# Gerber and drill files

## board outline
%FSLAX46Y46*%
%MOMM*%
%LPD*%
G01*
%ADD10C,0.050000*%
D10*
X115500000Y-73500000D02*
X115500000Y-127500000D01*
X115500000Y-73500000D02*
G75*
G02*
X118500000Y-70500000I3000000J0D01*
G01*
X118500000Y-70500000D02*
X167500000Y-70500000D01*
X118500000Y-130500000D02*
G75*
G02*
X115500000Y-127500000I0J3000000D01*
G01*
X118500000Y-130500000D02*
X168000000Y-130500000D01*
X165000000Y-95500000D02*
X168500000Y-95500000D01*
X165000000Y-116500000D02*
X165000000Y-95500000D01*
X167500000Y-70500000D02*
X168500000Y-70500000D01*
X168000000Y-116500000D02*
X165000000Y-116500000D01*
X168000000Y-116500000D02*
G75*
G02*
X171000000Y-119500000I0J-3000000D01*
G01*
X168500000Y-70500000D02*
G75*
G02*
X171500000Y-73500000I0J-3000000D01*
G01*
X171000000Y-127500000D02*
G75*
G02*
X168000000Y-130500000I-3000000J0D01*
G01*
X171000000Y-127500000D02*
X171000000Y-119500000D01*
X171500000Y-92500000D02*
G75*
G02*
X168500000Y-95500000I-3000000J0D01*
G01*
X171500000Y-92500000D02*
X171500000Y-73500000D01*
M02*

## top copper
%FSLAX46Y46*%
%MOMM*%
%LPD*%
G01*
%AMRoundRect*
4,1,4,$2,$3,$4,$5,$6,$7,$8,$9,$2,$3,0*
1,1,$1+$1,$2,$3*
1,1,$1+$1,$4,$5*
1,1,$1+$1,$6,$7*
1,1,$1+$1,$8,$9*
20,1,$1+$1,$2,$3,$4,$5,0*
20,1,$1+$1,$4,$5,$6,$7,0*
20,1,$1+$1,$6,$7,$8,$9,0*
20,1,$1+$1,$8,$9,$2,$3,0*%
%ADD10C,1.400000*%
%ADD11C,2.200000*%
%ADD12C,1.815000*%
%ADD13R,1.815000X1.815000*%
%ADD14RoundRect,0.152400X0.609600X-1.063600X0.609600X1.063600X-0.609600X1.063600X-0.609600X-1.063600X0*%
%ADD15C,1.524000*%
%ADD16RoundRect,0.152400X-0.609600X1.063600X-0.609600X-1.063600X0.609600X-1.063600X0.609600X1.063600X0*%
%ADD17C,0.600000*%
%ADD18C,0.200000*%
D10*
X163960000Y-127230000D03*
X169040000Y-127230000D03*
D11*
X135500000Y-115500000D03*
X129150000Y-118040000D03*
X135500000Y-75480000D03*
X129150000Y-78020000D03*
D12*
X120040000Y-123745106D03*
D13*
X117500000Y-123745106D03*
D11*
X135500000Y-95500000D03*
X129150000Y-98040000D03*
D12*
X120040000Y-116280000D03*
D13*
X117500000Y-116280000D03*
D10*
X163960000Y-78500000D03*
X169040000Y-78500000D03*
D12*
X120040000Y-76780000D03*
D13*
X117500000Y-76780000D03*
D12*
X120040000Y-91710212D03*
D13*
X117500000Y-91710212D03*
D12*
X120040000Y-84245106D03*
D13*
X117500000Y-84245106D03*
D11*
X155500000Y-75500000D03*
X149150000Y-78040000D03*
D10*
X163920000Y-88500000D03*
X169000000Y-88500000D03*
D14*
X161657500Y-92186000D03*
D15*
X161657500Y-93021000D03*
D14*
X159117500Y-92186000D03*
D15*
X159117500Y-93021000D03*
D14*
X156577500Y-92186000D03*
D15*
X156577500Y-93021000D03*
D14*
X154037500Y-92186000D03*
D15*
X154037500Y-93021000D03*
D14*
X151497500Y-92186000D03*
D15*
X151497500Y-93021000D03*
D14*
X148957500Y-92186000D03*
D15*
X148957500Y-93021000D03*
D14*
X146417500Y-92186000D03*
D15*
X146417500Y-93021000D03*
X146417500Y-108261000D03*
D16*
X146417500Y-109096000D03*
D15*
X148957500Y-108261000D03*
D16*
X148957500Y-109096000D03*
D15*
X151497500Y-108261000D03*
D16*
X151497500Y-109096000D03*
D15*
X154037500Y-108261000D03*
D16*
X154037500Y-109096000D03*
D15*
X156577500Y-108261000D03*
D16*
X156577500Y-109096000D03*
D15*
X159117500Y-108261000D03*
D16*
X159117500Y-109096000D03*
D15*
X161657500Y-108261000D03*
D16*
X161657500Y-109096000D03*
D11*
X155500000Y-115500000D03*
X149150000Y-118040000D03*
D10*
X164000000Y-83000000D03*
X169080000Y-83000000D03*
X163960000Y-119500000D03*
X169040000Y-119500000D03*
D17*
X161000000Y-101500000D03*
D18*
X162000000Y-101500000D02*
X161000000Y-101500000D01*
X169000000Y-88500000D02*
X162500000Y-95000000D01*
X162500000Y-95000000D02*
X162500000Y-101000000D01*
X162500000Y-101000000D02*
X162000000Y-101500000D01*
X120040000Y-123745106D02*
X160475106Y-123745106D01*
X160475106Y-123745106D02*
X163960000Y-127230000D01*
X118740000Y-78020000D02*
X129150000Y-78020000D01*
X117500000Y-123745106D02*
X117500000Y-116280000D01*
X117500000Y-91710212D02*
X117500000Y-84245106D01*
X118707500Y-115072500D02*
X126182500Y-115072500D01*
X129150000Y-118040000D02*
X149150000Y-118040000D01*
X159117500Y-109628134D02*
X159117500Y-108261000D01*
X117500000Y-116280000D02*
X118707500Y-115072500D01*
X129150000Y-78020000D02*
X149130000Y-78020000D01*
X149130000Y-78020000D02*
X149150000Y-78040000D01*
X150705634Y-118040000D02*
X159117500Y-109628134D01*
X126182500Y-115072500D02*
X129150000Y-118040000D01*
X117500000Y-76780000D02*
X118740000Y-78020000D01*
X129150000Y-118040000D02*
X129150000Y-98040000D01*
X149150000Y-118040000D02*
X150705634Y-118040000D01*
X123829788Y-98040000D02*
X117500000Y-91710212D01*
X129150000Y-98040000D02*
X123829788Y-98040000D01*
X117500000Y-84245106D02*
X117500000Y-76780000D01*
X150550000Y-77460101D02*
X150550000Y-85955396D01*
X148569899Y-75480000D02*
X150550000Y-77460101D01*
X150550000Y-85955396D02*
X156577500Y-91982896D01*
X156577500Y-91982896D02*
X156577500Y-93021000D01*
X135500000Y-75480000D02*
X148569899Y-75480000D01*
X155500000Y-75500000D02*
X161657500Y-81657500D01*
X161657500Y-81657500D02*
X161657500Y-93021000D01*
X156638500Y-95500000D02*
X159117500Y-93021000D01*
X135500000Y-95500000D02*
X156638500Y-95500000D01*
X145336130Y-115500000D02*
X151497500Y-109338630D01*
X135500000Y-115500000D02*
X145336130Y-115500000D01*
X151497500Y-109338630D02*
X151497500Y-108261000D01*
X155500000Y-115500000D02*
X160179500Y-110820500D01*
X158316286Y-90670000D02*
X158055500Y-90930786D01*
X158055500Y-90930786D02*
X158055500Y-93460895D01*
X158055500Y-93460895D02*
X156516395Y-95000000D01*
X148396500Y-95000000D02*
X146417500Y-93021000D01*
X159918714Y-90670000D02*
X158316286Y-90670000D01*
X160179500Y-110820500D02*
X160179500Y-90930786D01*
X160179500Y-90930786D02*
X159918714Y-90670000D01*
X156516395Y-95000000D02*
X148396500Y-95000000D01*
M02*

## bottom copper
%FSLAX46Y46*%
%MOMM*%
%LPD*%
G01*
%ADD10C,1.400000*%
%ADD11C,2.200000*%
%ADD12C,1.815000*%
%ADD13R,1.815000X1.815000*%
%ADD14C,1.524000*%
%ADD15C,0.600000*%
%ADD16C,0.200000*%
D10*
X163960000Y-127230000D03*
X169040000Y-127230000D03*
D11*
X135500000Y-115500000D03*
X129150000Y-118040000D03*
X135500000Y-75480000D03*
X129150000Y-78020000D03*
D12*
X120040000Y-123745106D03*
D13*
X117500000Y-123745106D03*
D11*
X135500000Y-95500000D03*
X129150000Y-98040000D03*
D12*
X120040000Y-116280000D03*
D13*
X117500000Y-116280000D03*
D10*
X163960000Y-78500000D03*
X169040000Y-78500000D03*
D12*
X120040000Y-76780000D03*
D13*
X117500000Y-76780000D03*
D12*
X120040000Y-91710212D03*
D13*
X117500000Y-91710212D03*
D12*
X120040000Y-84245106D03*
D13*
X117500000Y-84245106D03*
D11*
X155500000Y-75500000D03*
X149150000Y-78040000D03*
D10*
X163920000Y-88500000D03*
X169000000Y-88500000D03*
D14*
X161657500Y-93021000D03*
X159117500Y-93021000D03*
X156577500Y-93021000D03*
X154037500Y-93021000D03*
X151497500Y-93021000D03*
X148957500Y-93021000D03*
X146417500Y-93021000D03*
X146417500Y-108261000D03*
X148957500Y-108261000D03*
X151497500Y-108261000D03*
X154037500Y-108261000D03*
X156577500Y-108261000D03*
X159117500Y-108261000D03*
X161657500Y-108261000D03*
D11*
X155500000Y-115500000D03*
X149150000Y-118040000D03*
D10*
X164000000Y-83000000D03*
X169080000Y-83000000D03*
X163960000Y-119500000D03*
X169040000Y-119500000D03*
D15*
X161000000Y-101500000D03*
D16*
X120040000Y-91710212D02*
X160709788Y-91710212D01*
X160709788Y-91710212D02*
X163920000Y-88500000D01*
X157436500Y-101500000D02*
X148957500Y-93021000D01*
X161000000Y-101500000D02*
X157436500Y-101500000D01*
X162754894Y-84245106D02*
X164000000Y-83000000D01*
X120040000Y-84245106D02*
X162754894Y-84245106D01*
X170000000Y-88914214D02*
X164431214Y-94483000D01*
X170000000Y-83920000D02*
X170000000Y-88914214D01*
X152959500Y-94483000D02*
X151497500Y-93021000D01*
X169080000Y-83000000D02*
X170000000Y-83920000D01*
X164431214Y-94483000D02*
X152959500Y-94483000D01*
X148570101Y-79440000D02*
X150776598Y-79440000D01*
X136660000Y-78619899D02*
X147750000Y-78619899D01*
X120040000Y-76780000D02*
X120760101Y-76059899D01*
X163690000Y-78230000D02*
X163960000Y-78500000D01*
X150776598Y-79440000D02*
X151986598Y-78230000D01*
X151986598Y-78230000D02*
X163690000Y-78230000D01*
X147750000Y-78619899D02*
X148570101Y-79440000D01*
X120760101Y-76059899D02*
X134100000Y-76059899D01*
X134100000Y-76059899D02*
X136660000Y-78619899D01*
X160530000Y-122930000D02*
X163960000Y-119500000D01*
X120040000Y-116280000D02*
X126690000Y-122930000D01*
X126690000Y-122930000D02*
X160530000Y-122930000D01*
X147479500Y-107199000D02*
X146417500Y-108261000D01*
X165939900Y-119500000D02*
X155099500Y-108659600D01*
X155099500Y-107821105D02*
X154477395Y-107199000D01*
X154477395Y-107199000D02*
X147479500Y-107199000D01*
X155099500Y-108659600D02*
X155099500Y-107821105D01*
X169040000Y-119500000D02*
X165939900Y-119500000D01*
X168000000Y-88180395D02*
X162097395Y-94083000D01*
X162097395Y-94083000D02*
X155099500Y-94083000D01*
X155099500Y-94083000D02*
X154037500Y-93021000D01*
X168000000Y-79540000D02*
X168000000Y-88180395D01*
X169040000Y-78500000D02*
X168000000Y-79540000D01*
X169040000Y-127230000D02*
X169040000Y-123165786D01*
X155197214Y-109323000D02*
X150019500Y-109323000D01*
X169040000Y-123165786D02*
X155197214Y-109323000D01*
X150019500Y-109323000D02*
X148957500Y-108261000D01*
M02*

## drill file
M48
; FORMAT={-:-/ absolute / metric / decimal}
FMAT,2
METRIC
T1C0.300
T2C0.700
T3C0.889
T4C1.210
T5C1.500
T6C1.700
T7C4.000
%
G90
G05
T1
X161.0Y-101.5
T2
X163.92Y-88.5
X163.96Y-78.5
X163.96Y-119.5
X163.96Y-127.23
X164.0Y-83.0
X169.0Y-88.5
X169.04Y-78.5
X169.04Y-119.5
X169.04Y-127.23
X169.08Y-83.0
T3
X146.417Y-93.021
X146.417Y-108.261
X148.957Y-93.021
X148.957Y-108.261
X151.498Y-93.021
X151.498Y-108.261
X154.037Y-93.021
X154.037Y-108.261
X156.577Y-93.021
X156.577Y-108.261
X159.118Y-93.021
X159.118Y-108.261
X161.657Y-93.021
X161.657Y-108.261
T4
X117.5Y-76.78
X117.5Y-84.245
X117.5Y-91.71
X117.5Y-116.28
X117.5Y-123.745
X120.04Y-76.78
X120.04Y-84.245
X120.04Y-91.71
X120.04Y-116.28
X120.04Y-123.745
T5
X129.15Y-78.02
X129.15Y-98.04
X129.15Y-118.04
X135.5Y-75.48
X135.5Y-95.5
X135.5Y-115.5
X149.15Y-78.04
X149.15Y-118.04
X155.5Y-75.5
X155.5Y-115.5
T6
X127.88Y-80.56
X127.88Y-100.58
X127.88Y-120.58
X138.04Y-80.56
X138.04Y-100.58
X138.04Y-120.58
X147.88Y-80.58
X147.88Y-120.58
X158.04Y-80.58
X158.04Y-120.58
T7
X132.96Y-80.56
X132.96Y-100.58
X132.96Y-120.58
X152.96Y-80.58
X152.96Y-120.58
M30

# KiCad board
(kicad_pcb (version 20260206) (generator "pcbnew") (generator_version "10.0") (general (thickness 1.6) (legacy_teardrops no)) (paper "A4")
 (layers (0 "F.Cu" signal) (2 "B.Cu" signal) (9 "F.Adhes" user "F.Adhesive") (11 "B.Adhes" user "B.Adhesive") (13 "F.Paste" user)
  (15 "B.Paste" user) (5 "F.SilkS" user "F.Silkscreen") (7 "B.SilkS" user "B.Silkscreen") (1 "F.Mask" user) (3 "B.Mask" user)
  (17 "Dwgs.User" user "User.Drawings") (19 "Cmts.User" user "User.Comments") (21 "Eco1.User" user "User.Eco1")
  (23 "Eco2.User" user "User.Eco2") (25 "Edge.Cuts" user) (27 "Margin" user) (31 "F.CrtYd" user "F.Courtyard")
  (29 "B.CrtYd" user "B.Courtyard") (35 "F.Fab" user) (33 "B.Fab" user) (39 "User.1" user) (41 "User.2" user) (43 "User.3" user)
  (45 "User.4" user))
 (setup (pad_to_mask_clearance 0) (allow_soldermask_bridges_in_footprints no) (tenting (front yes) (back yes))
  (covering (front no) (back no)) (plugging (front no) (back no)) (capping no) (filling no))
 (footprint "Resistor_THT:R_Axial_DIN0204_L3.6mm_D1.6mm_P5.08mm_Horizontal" (layer "F.Cu") (at 163.96 127.23)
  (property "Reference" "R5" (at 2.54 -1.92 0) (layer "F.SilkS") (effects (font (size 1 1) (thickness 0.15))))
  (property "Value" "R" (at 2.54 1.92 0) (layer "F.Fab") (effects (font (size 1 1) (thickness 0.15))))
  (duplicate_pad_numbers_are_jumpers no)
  (pad "1" thru_hole circle (at 0 0) (size 1.4 1.4) (drill 0.7) (layers "*.Cu" "*.Mask") (remove_unused_layers no) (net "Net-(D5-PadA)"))
  (pad "2" thru_hole circle (at 5.08 0) (size 1.4 1.4) (drill 0.7) (layers "*.Cu" "*.Mask") (remove_unused_layers no)
   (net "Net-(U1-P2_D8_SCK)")))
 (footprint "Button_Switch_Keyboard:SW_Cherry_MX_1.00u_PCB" (layer "F.Cu") (at 135.5 115.5)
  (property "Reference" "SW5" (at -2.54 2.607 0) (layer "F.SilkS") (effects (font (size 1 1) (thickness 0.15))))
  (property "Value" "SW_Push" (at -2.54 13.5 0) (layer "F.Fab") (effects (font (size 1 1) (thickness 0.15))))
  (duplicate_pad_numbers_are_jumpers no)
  (pad "" np_thru_hole circle (at -7.62 5.08) (size 1.7 1.7) (drill 1.7) (layers "*.Cu" "*.Mask"))
  (pad "" np_thru_hole circle (at -2.54 5.08) (size 4 4) (drill 4) (layers "*.Cu" "*.Mask"))
  (pad "" np_thru_hole circle (at 2.54 5.08) (size 1.7 1.7) (drill 1.7) (layers "*.Cu" "*.Mask"))
  (pad "1" thru_hole circle (at 0 0) (size 2.2 2.2) (drill 1.5) (layers "*.Cu" "*.Mask") (remove_unused_layers no)
   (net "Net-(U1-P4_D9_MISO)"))
  (pad "2" thru_hole circle (at -6.35 2.54) (size 2.2 2.2) (drill 1.5) (layers "*.Cu" "*.Mask") (remove_unused_layers no) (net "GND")))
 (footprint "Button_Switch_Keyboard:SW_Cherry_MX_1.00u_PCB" (layer "F.Cu") (at 135.5 75.48)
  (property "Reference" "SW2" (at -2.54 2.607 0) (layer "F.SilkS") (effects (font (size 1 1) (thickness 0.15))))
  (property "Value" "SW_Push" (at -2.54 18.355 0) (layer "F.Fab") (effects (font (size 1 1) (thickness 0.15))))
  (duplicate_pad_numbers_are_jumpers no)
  (pad "" np_thru_hole circle (at -7.62 5.08) (size 1.7 1.7) (drill 1.7) (layers "*.Cu" "*.Mask"))
  (pad "" np_thru_hole circle (at -2.54 5.08) (size 4 4) (drill 4) (layers "*.Cu" "*.Mask"))
  (pad "" np_thru_hole circle (at 2.54 5.08) (size 1.7 1.7) (drill 1.7) (layers "*.Cu" "*.Mask"))
  (pad "1" thru_hole circle (at 0 0) (size 2.2 2.2) (drill 1.5) (layers "*.Cu" "*.Mask") (remove_unused_layers no)
   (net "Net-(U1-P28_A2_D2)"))
  (pad "2" thru_hole circle (at -6.35 2.54) (size 2.2 2.2) (drill 1.5) (layers "*.Cu" "*.Mask") (remove_unused_layers no) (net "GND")))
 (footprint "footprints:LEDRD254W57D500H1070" (layer "F.Cu") (at 118.77 123.745106)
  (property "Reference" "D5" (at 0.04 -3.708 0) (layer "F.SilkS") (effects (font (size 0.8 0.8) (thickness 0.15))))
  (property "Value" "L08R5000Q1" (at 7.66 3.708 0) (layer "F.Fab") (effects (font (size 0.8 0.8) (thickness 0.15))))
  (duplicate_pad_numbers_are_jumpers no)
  (pad "A" thru_hole circle (at 1.27 0) (size 1.815 1.815) (drill 1.21) (layers "*.Cu" "*.Mask") (remove_unused_layers no)
   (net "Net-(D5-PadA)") (solder_mask_margin 0.102))
  (pad "C" thru_hole rect (at -1.27 0) (size 1.815 1.815) (drill 1.21) (layers "*.Cu" "*.Mask") (remove_unused_layers no) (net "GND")
   (solder_mask_margin 0.102)))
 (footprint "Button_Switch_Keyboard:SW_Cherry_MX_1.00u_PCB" (layer "F.Cu") (at 135.5 95.5)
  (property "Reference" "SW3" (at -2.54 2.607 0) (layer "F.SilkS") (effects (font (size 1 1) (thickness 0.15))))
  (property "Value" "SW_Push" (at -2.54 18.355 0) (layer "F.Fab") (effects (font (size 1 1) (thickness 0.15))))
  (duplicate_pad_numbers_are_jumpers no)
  (pad "" np_thru_hole circle (at -7.62 5.08) (size 1.7 1.7) (drill 1.7) (layers "*.Cu" "*.Mask"))
  (pad "" np_thru_hole circle (at -2.54 5.08) (size 4 4) (drill 4) (layers "*.Cu" "*.Mask"))
  (pad "" np_thru_hole circle (at 2.54 5.08) (size 1.7 1.7) (drill 1.7) (layers "*.Cu" "*.Mask"))
  (pad "1" thru_hole circle (at 0 0) (size 2.2 2.2) (drill 1.5) (layers "*.Cu" "*.Mask") (remove_unused_layers no)
   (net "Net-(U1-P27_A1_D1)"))
  (pad "2" thru_hole circle (at -6.35 2.54) (size 2.2 2.2) (drill 1.5) (layers "*.Cu" "*.Mask") (remove_unused_layers no) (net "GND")))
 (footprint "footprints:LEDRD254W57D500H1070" (layer "F.Cu") (at 118.77 116.28)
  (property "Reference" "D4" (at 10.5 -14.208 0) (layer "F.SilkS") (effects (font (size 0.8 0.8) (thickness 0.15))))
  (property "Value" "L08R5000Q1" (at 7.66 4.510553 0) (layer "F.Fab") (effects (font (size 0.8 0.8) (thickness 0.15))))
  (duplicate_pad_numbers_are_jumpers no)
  (pad "A" thru_hole circle (at 1.27 0) (size 1.815 1.815) (drill 1.21) (layers "*.Cu" "*.Mask") (remove_unused_layers no)
   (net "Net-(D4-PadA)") (solder_mask_margin 0.102))
  (pad "C" thru_hole rect (at -1.27 0) (size 1.815 1.815) (drill 1.21) (layers "*.Cu" "*.Mask") (remove_unused_layers no) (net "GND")
   (solder_mask_margin 0.102)))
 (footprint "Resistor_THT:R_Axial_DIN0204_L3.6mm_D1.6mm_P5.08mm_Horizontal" (layer "F.Cu") (at 163.96 78.5)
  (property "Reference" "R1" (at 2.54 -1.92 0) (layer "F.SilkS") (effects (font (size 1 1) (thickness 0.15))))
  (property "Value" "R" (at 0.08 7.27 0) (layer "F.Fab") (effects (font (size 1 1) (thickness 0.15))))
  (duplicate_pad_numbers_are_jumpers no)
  (pad "1" thru_hole circle (at 0 0) (size 1.4 1.4) (drill 0.7) (layers "*.Cu" "*.Mask") (remove_unused_layers no) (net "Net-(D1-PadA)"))
  (pad "2" thru_hole circle (at 5.08 0) (size 1.4 1.4) (drill 0.7) (layers "*.Cu" "*.Mask") (remove_unused_layers no)
   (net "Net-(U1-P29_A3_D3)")))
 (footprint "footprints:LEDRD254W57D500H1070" (layer "F.Cu") (at 118.77 76.78)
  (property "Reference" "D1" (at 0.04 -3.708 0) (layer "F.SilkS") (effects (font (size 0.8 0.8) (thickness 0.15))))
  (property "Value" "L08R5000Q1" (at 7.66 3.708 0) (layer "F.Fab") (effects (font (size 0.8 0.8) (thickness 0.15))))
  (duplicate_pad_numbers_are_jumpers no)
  (pad "A" thru_hole circle (at 1.27 0) (size 1.815 1.815) (drill 1.21) (layers "*.Cu" "*.Mask") (remove_unused_layers no)
   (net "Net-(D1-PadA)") (solder_mask_margin 0.102))
  (pad "C" thru_hole rect (at -1.27 0) (size 1.815 1.815) (drill 1.21) (layers "*.Cu" "*.Mask") (remove_unused_layers no) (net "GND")
   (solder_mask_margin 0.102)))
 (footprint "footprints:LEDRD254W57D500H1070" (layer "F.Cu") (at 118.77 91.710212)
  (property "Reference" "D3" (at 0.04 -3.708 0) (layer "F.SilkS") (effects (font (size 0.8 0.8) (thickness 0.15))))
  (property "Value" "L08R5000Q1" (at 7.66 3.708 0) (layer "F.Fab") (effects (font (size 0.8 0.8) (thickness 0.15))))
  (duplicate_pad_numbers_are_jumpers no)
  (pad "A" thru_hole circle (at 1.27 0) (size 1.815 1.815) (drill 1.21) (layers "*.Cu" "*.Mask") (remove_unused_layers no)
   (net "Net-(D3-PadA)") (solder_mask_margin 0.102))
  (pad "C" thru_hole rect (at -1.27 0) (size 1.815 1.815) (drill 1.21) (layers "*.Cu" "*.Mask") (remove_unused_layers no) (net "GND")
   (solder_mask_margin 0.102)))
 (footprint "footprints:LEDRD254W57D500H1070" (layer "F.Cu") (at 118.77 84.245106)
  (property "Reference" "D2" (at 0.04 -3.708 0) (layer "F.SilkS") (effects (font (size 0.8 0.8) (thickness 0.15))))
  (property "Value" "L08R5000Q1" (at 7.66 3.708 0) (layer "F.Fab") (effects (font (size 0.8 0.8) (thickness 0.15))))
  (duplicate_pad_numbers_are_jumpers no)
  (pad "A" thru_hole circle (at 1.27 0) (size 1.815 1.815) (drill 1.21) (layers "*.Cu" "*.Mask") (remove_unused_layers no)
   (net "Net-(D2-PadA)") (solder_mask_margin 0.102))
  (pad "C" thru_hole rect (at -1.27 0) (size 1.815 1.815) (drill 1.21) (layers "*.Cu" "*.Mask") (remove_unused_layers no) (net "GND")
   (solder_mask_margin 0.102)))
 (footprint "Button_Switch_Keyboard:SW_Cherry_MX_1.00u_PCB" (layer "F.Cu") (at 155.5 75.5)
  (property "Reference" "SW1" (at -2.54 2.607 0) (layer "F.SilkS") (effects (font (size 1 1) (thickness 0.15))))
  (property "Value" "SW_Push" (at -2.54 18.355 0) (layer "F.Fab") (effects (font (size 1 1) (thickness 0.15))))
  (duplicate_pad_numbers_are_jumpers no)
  (pad "" np_thru_hole circle (at -7.62 5.08) (size 1.7 1.7) (drill 1.7) (layers "*.Cu" "*.Mask"))
  (pad "" np_thru_hole circle (at -2.54 5.08) (size 4 4) (drill 4) (layers "*.Cu" "*.Mask"))
  (pad "" np_thru_hole circle (at 2.54 5.08) (size 1.7 1.7) (drill 1.7) (layers "*.Cu" "*.Mask"))
  (pad "1" thru_hole circle (at 0 0) (size 2.2 2.2) (drill 1.5) (layers "*.Cu" "*.Mask") (remove_unused_layers no)
   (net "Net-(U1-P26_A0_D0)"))
  (pad "2" thru_hole circle (at -6.35 2.54) (size 2.2 2.2) (drill 1.5) (layers "*.Cu" "*.Mask") (remove_unused_layers no) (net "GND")))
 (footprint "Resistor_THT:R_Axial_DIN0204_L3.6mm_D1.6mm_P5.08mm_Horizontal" (layer "F.Cu") (at 163.92 88.5)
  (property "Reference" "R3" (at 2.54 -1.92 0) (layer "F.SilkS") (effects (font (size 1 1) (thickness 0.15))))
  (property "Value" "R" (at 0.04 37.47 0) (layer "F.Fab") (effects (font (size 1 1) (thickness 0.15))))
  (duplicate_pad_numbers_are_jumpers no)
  (pad "1" thru_hole circle (at 0 0) (size 1.4 1.4) (drill 0.7) (layers "*.Cu" "*.Mask") (remove_unused_layers no) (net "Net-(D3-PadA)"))
  (pad "2" thru_hole circle (at 5.08 0) (size 1.4 1.4) (drill 0.7) (layers "*.Cu" "*.Mask") (remove_unused_layers no)
   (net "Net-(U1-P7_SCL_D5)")))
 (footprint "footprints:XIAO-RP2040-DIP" (layer "F.Cu") (at 154.0375 100.641)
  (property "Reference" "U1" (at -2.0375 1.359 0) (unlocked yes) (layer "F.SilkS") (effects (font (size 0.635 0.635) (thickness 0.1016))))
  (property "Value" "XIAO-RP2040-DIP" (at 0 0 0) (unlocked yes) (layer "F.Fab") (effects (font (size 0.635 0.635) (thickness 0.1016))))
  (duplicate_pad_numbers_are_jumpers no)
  (pad "1" smd roundrect (at 7.62 -8.455 90) (size 2.432 1.524) (layers "F.Cu" "F.Mask") (roundrect_rratio 0.1) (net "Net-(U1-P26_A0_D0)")
   (thermal_bridge_angle 45))
  (pad "1" thru_hole circle (at 7.62 -7.62 90) (size 1.524 1.524) (drill 0.889) (layers "*.Cu" "*.Mask") (remove_unused_layers no)
   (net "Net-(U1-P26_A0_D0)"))
  (pad "2" smd roundrect (at 5.08 -8.455 90) (size 2.432 1.524) (layers "F.Cu" "F.Mask") (roundrect_rratio 0.1) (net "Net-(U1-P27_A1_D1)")
   (thermal_bridge_angle 45))
  (pad "2" thru_hole circle (at 5.08 -7.62 90) (size 1.524 1.524) (drill 0.889) (layers "*.Cu" "*.Mask") (remove_unused_layers no)
   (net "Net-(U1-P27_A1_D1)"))
  (pad "3" smd roundrect (at 2.54 -8.455 90) (size 2.432 1.524) (layers "F.Cu" "F.Mask") (roundrect_rratio 0.1) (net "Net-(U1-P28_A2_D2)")
   (thermal_bridge_angle 45))
  (pad "3" thru_hole circle (at 2.54 -7.62 90) (size 1.524 1.524) (drill 0.889) (layers "*.Cu" "*.Mask") (remove_unused_layers no)
   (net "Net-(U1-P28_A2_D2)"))
  (pad "4" smd roundrect (at 0 -8.455 90) (size 2.432 1.524) (layers "F.Cu" "F.Mask") (roundrect_rratio 0.1) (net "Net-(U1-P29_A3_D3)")
   (thermal_bridge_angle 45))
  (pad "4" thru_hole circle (at 0 -7.62 90) (size 1.524 1.524) (drill 0.889) (layers "*.Cu" "*.Mask") (remove_unused_layers no)
   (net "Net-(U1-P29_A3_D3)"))
  (pad "5" smd roundrect (at -2.54 -8.455 90) (size 2.432 1.524) (layers "F.Cu" "F.Mask") (roundrect_rratio 0.1) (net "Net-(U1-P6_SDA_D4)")
   (thermal_bridge_angle 45))
  (pad "5" thru_hole circle (at -2.54 -7.62 90) (size 1.524 1.524) (drill 0.889) (layers "*.Cu" "*.Mask") (remove_unused_layers no)
   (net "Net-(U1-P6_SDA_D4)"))
  (pad "6" smd roundrect (at -5.08 -8.455 90) (size 2.432 1.524) (layers "F.Cu" "F.Mask") (roundrect_rratio 0.1) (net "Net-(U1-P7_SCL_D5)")
   (thermal_bridge_angle 45))
  (pad "6" thru_hole circle (at -5.08 -7.62 90) (size 1.524 1.524) (drill 0.889) (layers "*.Cu" "*.Mask") (remove_unused_layers no)
   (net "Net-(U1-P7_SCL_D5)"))
  (pad "7" smd roundrect (at -7.62 -8.455 90) (size 2.432 1.524) (layers "F.Cu" "F.Mask") (roundrect_rratio 0.1) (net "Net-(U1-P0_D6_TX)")
   (thermal_bridge_angle 45))
  (pad "7" thru_hole circle (at -7.62 -7.62 90) (size 1.524 1.524) (drill 0.889) (layers "*.Cu" "*.Mask") (remove_unused_layers no)
   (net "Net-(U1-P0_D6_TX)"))
  (pad "8" thru_hole circle (at -7.62 7.62 270) (size 1.524 1.524) (drill 0.889) (layers "*.Cu" "*.Mask") (remove_unused_layers no)
   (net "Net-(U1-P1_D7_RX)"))
  (pad "8" smd roundrect (at -7.62 8.455 270) (size 2.432 1.524) (layers "F.Cu" "F.Mask") (roundrect_rratio 0.1) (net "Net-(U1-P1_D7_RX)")
   (thermal_bridge_angle 45))
  (pad "9" thru_hole circle (at -5.08 7.62 270) (size 1.524 1.524) (drill 0.889) (layers "*.Cu" "*.Mask") (remove_unused_layers no)
   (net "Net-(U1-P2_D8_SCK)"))
  (pad "9" smd roundrect (at -5.08 8.455 270) (size 2.432 1.524) (layers "F.Cu" "F.Mask") (roundrect_rratio 0.1) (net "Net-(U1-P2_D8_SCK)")
   (thermal_bridge_angle 45))
  (pad "10" thru_hole circle (at -2.54 7.62 270) (size 1.524 1.524) (drill 0.889) (layers "*.Cu" "*.Mask") (remove_unused_layers no)
   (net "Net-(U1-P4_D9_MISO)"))
  (pad "10" smd roundrect (at -2.54 8.455 270) (size 2.432 1.524) (layers "F.Cu" "F.Mask") (roundrect_rratio 0.1)
   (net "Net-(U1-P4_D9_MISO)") (thermal_bridge_angle 45))
  (pad "11" thru_hole circle (at 0 7.62 270) (size 1.524 1.524) (drill 0.889) (layers "*.Cu" "*.Mask") (remove_unused_layers no)
   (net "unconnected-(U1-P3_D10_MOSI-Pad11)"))
  (pad "11" smd roundrect (at 0 8.455 270) (size 2.432 1.524) (layers "F.Cu" "F.Mask") (roundrect_rratio 0.1)
   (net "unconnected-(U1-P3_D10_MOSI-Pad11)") (thermal_bridge_angle 45))
  (pad "12" thru_hole circle (at 2.54 7.62 270) (size 1.524 1.524) (drill 0.889) (layers "*.Cu" "*.Mask") (remove_unused_layers no)
   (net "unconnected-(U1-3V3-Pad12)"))
  (pad "12" smd roundrect (at 2.54 8.455 270) (size 2.432 1.524) (layers "F.Cu" "F.Mask") (roundrect_rratio 0.1)
   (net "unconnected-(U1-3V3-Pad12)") (thermal_bridge_angle 45))
  (pad "13" thru_hole circle (at 5.08 7.62 270) (size 1.524 1.524) (drill 0.889) (layers "*.Cu" "*.Mask") (remove_unused_layers no)
   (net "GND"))
  (pad "13" smd roundrect (at 5.08 8.455 270) (size 2.432 1.524) (layers "F.Cu" "F.Mask") (roundrect_rratio 0.1) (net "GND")
   (thermal_bridge_angle 45))
  (pad "14" thru_hole circle (at 7.62 7.62 270) (size 1.524 1.524) (drill 0.889) (layers "*.Cu" "*.Mask") (remove_unused_layers no)
   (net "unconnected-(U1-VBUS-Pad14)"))
  (pad "14" smd roundrect (at 7.62 8.455 270) (size 2.432 1.524) (layers "F.Cu" "F.Mask") (roundrect_rratio 0.1)
   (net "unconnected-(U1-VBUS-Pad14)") (thermal_bridge_angle 45)))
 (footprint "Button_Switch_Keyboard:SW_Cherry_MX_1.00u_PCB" (layer "F.Cu") (at 155.5 115.5)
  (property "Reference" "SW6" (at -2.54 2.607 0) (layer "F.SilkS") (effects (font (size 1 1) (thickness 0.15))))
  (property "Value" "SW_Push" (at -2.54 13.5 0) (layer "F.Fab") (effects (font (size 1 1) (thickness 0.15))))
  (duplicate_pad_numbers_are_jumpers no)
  (pad "" np_thru_hole circle (at -7.62 5.08) (size 1.7 1.7) (drill 1.7) (layers "*.Cu" "*.Mask"))
  (pad "" np_thru_hole circle (at -2.54 5.08) (size 4 4) (drill 4) (layers "*.Cu" "*.Mask"))
  (pad "" np_thru_hole circle (at 2.54 5.08) (size 1.7 1.7) (drill 1.7) (layers "*.Cu" "*.Mask"))
  (pad "1" thru_hole circle (at 0 0) (size 2.2 2.2) (drill 1.5) (layers "*.Cu" "*.Mask") (remove_unused_layers no) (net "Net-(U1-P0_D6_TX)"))
  (pad "2" thru_hole circle (at -6.35 2.54) (size 2.2 2.2) (drill 1.5) (layers "*.Cu" "*.Mask") (remove_unused_layers no) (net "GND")))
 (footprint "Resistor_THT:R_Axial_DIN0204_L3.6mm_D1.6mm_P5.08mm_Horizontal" (layer "F.Cu") (at 164 83)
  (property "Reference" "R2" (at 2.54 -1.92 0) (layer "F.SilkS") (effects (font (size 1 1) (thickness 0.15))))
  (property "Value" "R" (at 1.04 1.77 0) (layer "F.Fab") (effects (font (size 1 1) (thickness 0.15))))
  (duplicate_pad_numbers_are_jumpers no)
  (pad "1" thru_hole circle (at 0 0) (size 1.4 1.4) (drill 0.7) (layers "*.Cu" "*.Mask") (remove_unused_layers no) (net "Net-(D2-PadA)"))
  (pad "2" thru_hole circle (at 5.08 0) (size 1.4 1.4) (drill 0.7) (layers "*.Cu" "*.Mask") (remove_unused_layers no)
   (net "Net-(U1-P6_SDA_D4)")))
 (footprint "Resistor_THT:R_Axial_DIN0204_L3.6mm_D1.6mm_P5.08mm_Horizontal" (layer "F.Cu") (at 163.96 119.5)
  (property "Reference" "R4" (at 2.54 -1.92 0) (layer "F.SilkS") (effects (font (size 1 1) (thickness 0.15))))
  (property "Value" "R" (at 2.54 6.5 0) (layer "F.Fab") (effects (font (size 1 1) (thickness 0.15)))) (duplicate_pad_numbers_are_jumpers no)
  (pad "1" thru_hole circle (at 0 0) (size 1.4 1.4) (drill 0.7) (layers "*.Cu" "*.Mask") (remove_unused_layers no) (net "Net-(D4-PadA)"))
  (pad "2" thru_hole circle (at 5.08 0) (size 1.4 1.4) (drill 0.7) (layers "*.Cu" "*.Mask") (remove_unused_layers no)
   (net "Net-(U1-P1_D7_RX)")))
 (gr_line (start 115.5 73.5) (end 115.5 127.5) (stroke (width 0.05) (type default)) (layer "Edge.Cuts"))
 (gr_arc (start 115.5 73.5) (mid 116.37868 71.37868) (end 118.5 70.5) (stroke (width 0.05) (type default)) (layer "Edge.Cuts"))
 (gr_line (start 118.5 70.5) (end 167.5 70.5) (stroke (width 0.05) (type default)) (layer "Edge.Cuts"))
 (gr_arc (start 118.5 130.5) (mid 116.37868 129.62132) (end 115.5 127.5) (stroke (width 0.05) (type default)) (layer "Edge.Cuts"))
 (gr_line (start 118.5 130.5) (end 168 130.5) (stroke (width 0.05) (type default)) (layer "Edge.Cuts"))
 (gr_line (start 165 95.5) (end 168.5 95.5) (stroke (width 0.05) (type default)) (layer "Edge.Cuts"))
 (gr_line (start 165 116.5) (end 165 95.5) (stroke (width 0.05) (type default)) (layer "Edge.Cuts"))
 (gr_line (start 167.5 70.5) (end 168.5 70.5) (stroke (width 0.05) (type default)) (layer "Edge.Cuts"))
 (gr_line (start 168 116.5) (end 165 116.5) (stroke (width 0.05) (type default)) (layer "Edge.Cuts"))
 (gr_arc (start 168 116.5) (mid 170.12132 117.37868) (end 171 119.5) (stroke (width 0.05) (type default)) (layer "Edge.Cuts"))
 (gr_arc (start 168.5 70.5) (mid 170.62132 71.37868) (end 171.5 73.5) (stroke (width 0.05) (type default)) (layer "Edge.Cuts"))
 (gr_arc (start 171 127.5) (mid 170.12132 129.62132) (end 168 130.5) (stroke (width 0.05) (type default)) (layer "Edge.Cuts"))
 (gr_line (start 171 127.5) (end 171 119.5) (stroke (width 0.05) (type default)) (layer "Edge.Cuts"))
 (gr_arc (start 171.5 92.5) (mid 170.62132 94.62132) (end 168.5 95.5) (stroke (width 0.05) (type default)) (layer "Edge.Cuts"))
 (gr_line (start 171.5 92.5) (end 171.5 73.5) (stroke (width 0.05) (type default)) (layer "Edge.Cuts"))
 (segment (start 120.04 91.710212) (end 160.709788 91.710212) (width 0.2) (layer "B.Cu") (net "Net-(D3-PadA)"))
 (segment (start 160.709788 91.710212) (end 163.92 88.5) (width 0.2) (layer "B.Cu") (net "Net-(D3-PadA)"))
 (segment (start 162 101.5) (end 161 101.5) (width 0.2) (layer "F.Cu") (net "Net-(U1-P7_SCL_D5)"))
 (segment (start 169 88.5) (end 162.5 95) (width 0.2) (layer "F.Cu") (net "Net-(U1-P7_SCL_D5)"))
 (segment (start 162.5 95) (end 162.5 101) (width 0.2) (layer "F.Cu") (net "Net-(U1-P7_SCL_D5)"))
 (segment (start 162.5 101) (end 162 101.5) (width 0.2) (layer "F.Cu") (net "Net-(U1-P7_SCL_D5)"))
 (via (at 161 101.5) (size 0.6) (drill 0.3) (layers "F.Cu" "B.Cu") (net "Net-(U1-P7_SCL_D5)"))
 (segment (start 157.4365 101.5) (end 148.9575 93.021) (width 0.2) (layer "B.Cu") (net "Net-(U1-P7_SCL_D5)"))
 (segment (start 161 101.5) (end 157.4365 101.5) (width 0.2) (layer "B.Cu") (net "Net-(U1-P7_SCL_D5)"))
 (segment (start 120.04 123.745106) (end 160.475106 123.745106) (width 0.2) (layer "F.Cu") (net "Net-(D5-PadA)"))
 (segment (start 160.475106 123.745106) (end 163.96 127.23) (width 0.2) (layer "F.Cu") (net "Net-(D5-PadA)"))
 (segment (start 118.74 78.02) (end 129.15 78.02) (width 0.2) (layer "F.Cu") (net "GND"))
 (segment (start 117.5 123.745106) (end 117.5 116.28) (width 0.2) (layer "F.Cu") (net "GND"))
 (segment (start 117.5 91.710212) (end 117.5 84.245106) (width 0.2) (layer "F.Cu") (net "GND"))
 (segment (start 118.7075 115.0725) (end 126.1825 115.0725) (width 0.2) (layer "F.Cu") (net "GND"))
 (segment (start 129.15 118.04) (end 149.15 118.04) (width 0.2) (layer "F.Cu") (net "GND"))
 (segment (start 159.1175 109.628134) (end 159.1175 108.261) (width 0.2) (layer "F.Cu") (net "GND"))
 (segment (start 117.5 116.28) (end 118.7075 115.0725) (width 0.2) (layer "F.Cu") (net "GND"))
 (segment (start 129.15 78.02) (end 149.13 78.02) (width 0.2) (layer "F.Cu") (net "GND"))
 (segment (start 149.13 78.02) (end 149.15 78.04) (width 0.2) (layer "F.Cu") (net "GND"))
 (segment (start 150.705634 118.04) (end 159.1175 109.628134) (width 0.2) (layer "F.Cu") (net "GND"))
 (segment (start 126.1825 115.0725) (end 129.15 118.04) (width 0.2) (layer "F.Cu") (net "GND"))
 (segment (start 117.5 76.78) (end 118.74 78.02) (width 0.2) (layer "F.Cu") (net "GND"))
 (segment (start 129.15 118.04) (end 129.15 98.04) (width 0.2) (layer "F.Cu") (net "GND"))
 (segment (start 149.15 118.04) (end 150.705634 118.04) (width 0.2) (layer "F.Cu") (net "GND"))
 (segment (start 123.829788 98.04) (end 117.5 91.710212) (width 0.2) (layer "F.Cu") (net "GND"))
 (segment (start 129.15 98.04) (end 123.829788 98.04) (width 0.2) (layer "F.Cu") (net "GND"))
 (segment (start 117.5 84.245106) (end 117.5 76.78) (width 0.2) (layer "F.Cu") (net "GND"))
 (segment (start 162.754894 84.245106) (end 164 83) (width 0.2) (layer "B.Cu") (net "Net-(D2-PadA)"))
 (segment (start 120.04 84.245106) (end 162.754894 84.245106) (width 0.2) (layer "B.Cu") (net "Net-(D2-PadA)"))
 (segment (start 170 88.914214) (end 164.431214 94.483) (width 0.2) (layer "B.Cu") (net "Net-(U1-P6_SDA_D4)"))
 (segment (start 170 83.92) (end 170 88.914214) (width 0.2) (layer "B.Cu") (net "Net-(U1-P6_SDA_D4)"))
 (segment (start 152.9595 94.483) (end 151.4975 93.021) (width 0.2) (layer "B.Cu") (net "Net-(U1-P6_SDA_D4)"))
 (segment (start 169.08 83) (end 170 83.92) (width 0.2) (layer "B.Cu") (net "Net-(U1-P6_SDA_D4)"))
 (segment (start 164.431214 94.483) (end 152.9595 94.483) (width 0.2) (layer "B.Cu") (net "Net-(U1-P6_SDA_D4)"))
 (segment (start 148.570101 79.44) (end 150.776598 79.44) (width 0.2) (layer "B.Cu") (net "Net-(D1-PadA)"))
 (segment (start 136.66 78.619899) (end 147.75 78.619899) (width 0.2) (layer "B.Cu") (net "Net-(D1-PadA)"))
 (segment (start 120.04 76.78) (end 120.760101 76.059899) (width 0.2) (layer "B.Cu") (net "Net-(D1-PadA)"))
 (segment (start 163.69 78.23) (end 163.96 78.5) (width 0.2) (layer "B.Cu") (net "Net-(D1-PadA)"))
 (segment (start 150.776598 79.44) (end 151.986598 78.23) (width 0.2) (layer "B.Cu") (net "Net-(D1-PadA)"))
 (segment (start 151.986598 78.23) (end 163.69 78.23) (width 0.2) (layer "B.Cu") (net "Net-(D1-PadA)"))
 (segment (start 147.75 78.619899) (end 148.570101 79.44) (width 0.2) (layer "B.Cu") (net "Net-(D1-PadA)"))
 (segment (start 120.760101 76.059899) (end 134.1 76.059899) (width 0.2) (layer "B.Cu") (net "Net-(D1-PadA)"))
 (segment (start 134.1 76.059899) (end 136.66 78.619899) (width 0.2) (layer "B.Cu") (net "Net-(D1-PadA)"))
 (segment (start 160.53 122.93) (end 163.96 119.5) (width 0.2) (layer "B.Cu") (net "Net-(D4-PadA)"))
 (segment (start 120.04 116.28) (end 126.69 122.93) (width 0.2) (layer "B.Cu") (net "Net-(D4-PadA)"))
 (segment (start 126.69 122.93) (end 160.53 122.93) (width 0.2) (layer "B.Cu") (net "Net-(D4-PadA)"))
 (segment (start 150.55 77.460101) (end 150.55 85.955396) (width 0.2) (layer "F.Cu") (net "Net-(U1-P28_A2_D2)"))
 (segment (start 148.569899 75.48) (end 150.55 77.460101) (width 0.2) (layer "F.Cu") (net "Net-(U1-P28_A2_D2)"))
 (segment (start 150.55 85.955396) (end 156.5775 91.982896) (width 0.2) (layer "F.Cu") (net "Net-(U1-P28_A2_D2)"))
 (segment (start 156.5775 91.982896) (end 156.5775 93.021) (width 0.2) (layer "F.Cu") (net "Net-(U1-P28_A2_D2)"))
 (segment (start 135.5 75.48) (end 148.569899 75.48) (width 0.2) (layer "F.Cu") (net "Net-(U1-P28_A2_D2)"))
 (segment (start 147.4795 107.199) (end 146.4175 108.261) (width 0.2) (layer "B.Cu") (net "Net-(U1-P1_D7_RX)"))
 (segment (start 165.9399 119.5) (end 155.0995 108.6596) (width 0.2) (layer "B.Cu") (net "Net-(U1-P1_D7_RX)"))
 (segment (start 155.0995 107.821105) (end 154.477395 107.199) (width 0.2) (layer "B.Cu") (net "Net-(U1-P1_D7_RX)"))
 (segment (start 154.477395 107.199) (end 147.4795 107.199) (width 0.2) (layer "B.Cu") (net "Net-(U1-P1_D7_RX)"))
 (segment (start 155.0995 108.6596) (end 155.0995 107.821105) (width 0.2) (layer "B.Cu") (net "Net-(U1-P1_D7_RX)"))
 (segment (start 169.04 119.5) (end 165.9399 119.5) (width 0.2) (layer "B.Cu") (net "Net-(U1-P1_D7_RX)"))
 (segment (start 155.5 75.5) (end 161.6575 81.6575) (width 0.2) (layer "F.Cu") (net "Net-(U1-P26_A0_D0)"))
 (segment (start 161.6575 81.6575) (end 161.6575 93.021) (width 0.2) (layer "F.Cu") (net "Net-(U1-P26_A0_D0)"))
 (segment (start 156.6385 95.5) (end 159.1175 93.021) (width 0.2) (layer "F.Cu") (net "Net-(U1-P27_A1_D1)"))
 (segment (start 135.5 95.5) (end 156.6385 95.5) (width 0.2) (layer "F.Cu") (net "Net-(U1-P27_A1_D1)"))
 (segment (start 145.33613 115.5) (end 151.4975 109.33863) (width 0.2) (layer "F.Cu") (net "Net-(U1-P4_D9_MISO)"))
 (segment (start 135.5 115.5) (end 145.33613 115.5) (width 0.2) (layer "F.Cu") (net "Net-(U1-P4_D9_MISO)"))
 (segment (start 151.4975 109.33863) (end 151.4975 108.261) (width 0.2) (layer "F.Cu") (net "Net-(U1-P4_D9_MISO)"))
 (segment (start 168 88.180395) (end 162.097395 94.083) (width 0.2) (layer "B.Cu") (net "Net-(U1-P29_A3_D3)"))
 (segment (start 162.097395 94.083) (end 155.0995 94.083) (width 0.2) (layer "B.Cu") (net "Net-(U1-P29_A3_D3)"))
 (segment (start 155.0995 94.083) (end 154.0375 93.021) (width 0.2) (layer "B.Cu") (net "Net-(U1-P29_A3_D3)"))
 (segment (start 168 79.54) (end 168 88.180395) (width 0.2) (layer "B.Cu") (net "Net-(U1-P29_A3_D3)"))
 (segment (start 169.04 78.5) (end 168 79.54) (width 0.2) (layer "B.Cu") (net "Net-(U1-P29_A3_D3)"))
 (segment (start 155.5 115.5) (end 160.1795 110.8205) (width 0.2) (layer "F.Cu") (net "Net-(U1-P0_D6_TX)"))
 (segment (start 158.316286 90.67) (end 158.0555 90.930786) (width 0.2) (layer "F.Cu") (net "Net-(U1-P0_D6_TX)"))
 (segment (start 158.0555 90.930786) (end 158.0555 93.460895) (width 0.2) (layer "F.Cu") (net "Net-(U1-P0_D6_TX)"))
 (segment (start 158.0555 93.460895) (end 156.516395 95) (width 0.2) (layer "F.Cu") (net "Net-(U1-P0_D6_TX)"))
 (segment (start 148.3965 95) (end 146.4175 93.021) (width 0.2) (layer "F.Cu") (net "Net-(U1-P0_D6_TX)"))
 (segment (start 159.918714 90.67) (end 158.316286 90.67) (width 0.2) (layer "F.Cu") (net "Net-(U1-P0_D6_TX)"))
 (segment (start 160.1795 110.8205) (end 160.1795 90.930786) (width 0.2) (layer "F.Cu") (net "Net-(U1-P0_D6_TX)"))
 (segment (start 160.1795 90.930786) (end 159.918714 90.67) (width 0.2) (layer "F.Cu") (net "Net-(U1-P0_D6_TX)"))
 (segment (start 156.516395 95) (end 148.3965 95) (width 0.2) (layer "F.Cu") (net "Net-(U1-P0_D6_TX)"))
 (segment (start 169.04 127.23) (end 169.04 123.165786) (width 0.2) (layer "B.Cu") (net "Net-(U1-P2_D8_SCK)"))
 (segment (start 155.197214 109.323) (end 150.0195 109.323) (width 0.2) (layer "B.Cu") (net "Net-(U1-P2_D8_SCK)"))
 (segment (start 169.04 123.165786) (end 155.197214 109.323) (width 0.2) (layer "B.Cu") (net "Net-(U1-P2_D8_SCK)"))
 (segment (start 150.0195 109.323) (end 148.9575 108.261) (width 0.2) (layer "B.Cu") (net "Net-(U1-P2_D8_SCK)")))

